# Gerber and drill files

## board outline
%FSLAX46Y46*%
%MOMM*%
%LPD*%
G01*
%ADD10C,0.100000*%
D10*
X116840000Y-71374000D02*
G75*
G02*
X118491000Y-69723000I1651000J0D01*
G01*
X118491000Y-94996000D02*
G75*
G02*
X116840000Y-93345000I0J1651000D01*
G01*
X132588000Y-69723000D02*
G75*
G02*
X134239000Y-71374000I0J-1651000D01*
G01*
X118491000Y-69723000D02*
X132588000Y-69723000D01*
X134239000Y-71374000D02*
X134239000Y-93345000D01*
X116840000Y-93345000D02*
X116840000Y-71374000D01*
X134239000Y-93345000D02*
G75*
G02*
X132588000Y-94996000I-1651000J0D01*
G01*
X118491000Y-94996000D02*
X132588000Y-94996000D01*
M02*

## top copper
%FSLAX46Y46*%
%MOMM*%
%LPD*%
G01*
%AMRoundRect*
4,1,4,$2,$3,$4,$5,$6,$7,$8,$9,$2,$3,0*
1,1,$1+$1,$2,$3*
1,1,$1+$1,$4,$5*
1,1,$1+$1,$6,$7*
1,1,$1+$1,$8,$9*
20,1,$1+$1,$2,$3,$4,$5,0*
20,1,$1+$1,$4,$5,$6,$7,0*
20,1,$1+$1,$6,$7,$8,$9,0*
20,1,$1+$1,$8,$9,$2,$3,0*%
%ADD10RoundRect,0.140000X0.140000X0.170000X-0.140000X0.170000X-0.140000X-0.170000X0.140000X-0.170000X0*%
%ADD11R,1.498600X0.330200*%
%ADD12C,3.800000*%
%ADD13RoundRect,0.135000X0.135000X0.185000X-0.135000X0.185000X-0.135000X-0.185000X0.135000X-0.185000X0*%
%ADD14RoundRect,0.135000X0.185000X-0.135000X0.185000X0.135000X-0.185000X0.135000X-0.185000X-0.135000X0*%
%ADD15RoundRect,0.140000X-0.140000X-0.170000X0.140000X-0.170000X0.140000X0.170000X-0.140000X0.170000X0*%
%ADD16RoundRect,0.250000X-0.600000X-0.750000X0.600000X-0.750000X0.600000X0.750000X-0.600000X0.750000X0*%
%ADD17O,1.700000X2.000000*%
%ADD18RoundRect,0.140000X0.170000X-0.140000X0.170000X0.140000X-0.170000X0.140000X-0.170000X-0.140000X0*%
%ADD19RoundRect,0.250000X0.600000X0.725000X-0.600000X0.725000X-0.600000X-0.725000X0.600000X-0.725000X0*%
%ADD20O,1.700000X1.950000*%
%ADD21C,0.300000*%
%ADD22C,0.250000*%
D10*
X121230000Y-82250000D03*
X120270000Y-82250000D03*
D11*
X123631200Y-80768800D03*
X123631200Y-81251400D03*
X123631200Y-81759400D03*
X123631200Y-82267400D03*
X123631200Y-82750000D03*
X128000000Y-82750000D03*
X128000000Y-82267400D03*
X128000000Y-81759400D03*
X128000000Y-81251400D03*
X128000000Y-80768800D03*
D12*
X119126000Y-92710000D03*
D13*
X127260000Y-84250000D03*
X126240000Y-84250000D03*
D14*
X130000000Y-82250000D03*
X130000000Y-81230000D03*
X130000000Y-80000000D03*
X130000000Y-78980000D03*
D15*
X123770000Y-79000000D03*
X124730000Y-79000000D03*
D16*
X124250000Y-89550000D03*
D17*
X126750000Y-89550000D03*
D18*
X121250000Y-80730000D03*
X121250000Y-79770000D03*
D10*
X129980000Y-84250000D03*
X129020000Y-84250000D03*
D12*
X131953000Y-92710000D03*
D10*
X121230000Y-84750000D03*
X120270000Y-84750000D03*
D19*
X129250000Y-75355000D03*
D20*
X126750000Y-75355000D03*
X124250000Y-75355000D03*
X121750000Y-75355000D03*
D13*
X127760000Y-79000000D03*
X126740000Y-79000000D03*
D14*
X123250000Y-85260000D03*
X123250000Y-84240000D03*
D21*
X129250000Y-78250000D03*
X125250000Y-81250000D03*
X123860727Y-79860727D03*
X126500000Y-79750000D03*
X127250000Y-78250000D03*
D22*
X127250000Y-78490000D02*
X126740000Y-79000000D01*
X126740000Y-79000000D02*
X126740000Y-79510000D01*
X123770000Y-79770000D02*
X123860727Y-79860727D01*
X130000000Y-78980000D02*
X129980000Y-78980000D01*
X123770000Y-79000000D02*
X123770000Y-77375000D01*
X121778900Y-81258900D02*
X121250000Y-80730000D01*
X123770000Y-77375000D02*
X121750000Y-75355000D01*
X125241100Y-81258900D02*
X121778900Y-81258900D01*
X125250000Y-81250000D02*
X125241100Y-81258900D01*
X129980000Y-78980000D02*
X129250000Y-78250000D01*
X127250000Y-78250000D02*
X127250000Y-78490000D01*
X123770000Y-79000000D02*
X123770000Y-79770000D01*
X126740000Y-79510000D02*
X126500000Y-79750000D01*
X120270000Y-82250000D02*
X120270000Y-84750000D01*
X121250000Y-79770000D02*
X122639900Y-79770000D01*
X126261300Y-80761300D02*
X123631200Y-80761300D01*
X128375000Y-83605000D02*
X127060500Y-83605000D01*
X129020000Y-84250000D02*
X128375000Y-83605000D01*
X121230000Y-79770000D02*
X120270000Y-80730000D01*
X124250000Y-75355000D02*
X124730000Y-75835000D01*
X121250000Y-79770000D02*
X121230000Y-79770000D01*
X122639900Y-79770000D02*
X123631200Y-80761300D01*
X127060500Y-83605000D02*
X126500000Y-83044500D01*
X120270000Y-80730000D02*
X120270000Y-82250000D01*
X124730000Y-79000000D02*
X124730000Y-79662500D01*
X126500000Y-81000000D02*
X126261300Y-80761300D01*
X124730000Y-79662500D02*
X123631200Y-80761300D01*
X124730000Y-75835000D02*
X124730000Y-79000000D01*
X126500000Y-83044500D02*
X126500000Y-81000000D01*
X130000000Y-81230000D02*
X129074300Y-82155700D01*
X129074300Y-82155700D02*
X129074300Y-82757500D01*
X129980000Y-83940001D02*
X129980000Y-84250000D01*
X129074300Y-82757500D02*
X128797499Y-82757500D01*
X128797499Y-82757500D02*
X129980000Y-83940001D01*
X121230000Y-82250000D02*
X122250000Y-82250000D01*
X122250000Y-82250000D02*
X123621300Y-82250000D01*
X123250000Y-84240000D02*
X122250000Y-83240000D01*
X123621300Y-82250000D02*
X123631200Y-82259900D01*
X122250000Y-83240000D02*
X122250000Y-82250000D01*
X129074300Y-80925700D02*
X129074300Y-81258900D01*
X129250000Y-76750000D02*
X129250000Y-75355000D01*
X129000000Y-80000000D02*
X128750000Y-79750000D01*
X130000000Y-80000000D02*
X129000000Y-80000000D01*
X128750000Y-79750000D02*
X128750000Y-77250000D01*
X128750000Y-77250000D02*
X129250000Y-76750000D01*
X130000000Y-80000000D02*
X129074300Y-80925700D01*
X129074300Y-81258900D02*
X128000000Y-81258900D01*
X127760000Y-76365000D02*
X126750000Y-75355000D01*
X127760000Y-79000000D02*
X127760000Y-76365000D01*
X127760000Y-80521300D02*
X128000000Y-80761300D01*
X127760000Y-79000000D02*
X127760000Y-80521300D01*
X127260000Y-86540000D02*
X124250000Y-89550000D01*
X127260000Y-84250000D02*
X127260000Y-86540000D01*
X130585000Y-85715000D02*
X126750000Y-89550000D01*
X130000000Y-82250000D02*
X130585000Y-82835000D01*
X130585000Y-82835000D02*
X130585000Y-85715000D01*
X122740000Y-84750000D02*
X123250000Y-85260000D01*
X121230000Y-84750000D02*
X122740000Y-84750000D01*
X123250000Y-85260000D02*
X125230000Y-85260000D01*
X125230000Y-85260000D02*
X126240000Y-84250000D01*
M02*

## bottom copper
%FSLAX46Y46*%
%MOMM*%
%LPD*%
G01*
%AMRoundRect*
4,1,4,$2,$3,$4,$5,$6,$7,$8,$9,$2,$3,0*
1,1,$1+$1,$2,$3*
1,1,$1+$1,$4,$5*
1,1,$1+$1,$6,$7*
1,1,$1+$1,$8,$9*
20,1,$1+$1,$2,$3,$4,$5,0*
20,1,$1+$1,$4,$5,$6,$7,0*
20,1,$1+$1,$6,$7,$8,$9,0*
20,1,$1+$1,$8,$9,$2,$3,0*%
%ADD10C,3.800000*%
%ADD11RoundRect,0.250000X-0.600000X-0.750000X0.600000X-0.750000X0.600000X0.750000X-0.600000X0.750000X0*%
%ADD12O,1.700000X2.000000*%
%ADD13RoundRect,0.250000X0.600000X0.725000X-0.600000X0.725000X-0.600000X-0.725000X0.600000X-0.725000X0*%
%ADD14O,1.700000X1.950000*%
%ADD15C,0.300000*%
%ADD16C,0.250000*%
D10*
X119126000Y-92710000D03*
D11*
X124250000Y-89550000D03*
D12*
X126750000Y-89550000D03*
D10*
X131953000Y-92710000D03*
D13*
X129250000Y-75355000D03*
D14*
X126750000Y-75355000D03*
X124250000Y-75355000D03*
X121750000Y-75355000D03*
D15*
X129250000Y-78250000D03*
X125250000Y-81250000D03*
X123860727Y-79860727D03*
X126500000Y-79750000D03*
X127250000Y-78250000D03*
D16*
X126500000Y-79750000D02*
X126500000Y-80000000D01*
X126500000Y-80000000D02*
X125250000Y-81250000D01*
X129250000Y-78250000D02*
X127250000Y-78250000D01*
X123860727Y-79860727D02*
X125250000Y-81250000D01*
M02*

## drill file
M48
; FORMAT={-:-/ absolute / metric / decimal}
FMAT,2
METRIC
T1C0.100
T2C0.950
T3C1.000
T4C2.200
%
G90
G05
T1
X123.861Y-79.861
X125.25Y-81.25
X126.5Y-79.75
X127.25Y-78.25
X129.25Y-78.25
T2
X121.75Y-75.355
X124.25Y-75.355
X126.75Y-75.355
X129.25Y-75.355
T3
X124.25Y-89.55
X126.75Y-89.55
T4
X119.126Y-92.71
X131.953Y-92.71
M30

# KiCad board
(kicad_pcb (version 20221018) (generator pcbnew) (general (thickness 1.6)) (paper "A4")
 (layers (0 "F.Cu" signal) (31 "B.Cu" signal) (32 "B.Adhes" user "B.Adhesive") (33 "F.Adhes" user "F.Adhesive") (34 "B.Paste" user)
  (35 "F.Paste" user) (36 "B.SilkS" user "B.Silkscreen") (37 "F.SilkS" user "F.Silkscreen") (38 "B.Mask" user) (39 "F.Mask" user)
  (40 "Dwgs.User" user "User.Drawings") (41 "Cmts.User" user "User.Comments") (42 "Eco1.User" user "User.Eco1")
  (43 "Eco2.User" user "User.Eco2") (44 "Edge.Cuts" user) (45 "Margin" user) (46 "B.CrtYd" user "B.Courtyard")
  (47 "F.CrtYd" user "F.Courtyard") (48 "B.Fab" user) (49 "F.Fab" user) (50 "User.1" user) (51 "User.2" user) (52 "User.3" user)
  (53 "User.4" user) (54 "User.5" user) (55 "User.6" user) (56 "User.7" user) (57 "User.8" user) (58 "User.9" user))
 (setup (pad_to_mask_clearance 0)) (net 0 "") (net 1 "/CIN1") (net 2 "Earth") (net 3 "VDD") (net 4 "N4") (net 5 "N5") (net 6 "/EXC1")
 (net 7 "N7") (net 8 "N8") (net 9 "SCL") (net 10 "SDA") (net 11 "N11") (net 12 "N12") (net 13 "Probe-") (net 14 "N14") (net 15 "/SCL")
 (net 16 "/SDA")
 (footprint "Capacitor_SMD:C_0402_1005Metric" (layer "F.Cu") (at 120.75 82.25 180)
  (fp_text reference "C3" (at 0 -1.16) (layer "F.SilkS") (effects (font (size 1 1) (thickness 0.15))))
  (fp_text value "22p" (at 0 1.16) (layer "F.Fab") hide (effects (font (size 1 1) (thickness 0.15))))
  (pad "1" smd roundrect (at -0.48 0 180) (size 0.56 0.62) (layers "F.Cu" "F.Paste" "F.Mask") (roundrect_rratio 0.25) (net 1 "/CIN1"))
  (pad "2" smd roundrect (at 0.48 0 180) (size 0.56 0.62) (layers "F.Cu" "F.Paste" "F.Mask") (roundrect_rratio 0.25) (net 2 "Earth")))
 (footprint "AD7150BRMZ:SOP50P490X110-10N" (layer "F.Cu") (at 125.8156 81.7594)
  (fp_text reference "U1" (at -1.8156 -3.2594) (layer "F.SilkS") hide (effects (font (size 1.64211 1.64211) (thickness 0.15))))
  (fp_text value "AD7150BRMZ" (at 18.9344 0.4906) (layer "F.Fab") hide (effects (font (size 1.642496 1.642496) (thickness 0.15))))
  (pad "1" smd rect (at -2.1844 -0.9906) (size 1.4986 0.3302) (layers "F.Cu" "F.Paste" "F.Mask") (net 2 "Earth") (solder_mask_margin 0.102))
  (pad "2" smd rect (at -2.1844 -0.508) (size 1.4986 0.3302) (layers "F.Cu" "F.Paste" "F.Mask") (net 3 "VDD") (solder_mask_margin 0.102))
  (pad "3" smd rect (at -2.1844 0) (size 1.4986 0.3302) (layers "F.Cu" "F.Paste" "F.Mask") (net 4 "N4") (solder_mask_margin 0.102))
  (pad "4" smd rect (at -2.1844 0.508) (size 1.4986 0.3302) (layers "F.Cu" "F.Paste" "F.Mask") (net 1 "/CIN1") (solder_mask_margin 0.102))
  (pad "5" smd rect (at -2.1844 0.9906) (size 1.4986 0.3302) (layers "F.Cu" "F.Paste" "F.Mask") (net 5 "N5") (solder_mask_margin 0.102))
  (pad "6" smd rect (at 2.1844 0.9906) (size 1.4986 0.3302) (layers "F.Cu" "F.Paste" "F.Mask") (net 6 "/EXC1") (solder_mask_margin 0.102))
  (pad "7" smd rect (at 2.1844 0.508) (size 1.4986 0.3302) (layers "F.Cu" "F.Paste" "F.Mask") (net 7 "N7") (solder_mask_margin 0.102))
  (pad "8" smd rect (at 2.1844 0) (size 1.4986 0.3302) (layers "F.Cu" "F.Paste" "F.Mask") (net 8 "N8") (solder_mask_margin 0.102))
  (pad "9" smd rect (at 2.1844 -0.508) (size 1.4986 0.3302) (layers "F.Cu" "F.Paste" "F.Mask") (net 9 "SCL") (solder_mask_margin 0.102))
  (pad "10" smd rect (at 2.1844 -0.9906) (size 1.4986 0.3302) (layers "F.Cu" "F.Paste" "F.Mask") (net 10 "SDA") (solder_mask_margin 0.102)))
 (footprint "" (layer "F.Cu") (at 119.126 92.71)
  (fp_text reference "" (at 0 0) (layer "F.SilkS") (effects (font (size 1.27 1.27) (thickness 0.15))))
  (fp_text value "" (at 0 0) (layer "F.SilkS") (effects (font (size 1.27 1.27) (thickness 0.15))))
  (pad "1" thru_hole circle (at 0 0 270) (size 3.8 3.8) (drill 2.2) (layers "*.Cu" "*.Mask")))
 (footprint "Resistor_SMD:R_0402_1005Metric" (layer "F.Cu") (at 126.75 84.25 180)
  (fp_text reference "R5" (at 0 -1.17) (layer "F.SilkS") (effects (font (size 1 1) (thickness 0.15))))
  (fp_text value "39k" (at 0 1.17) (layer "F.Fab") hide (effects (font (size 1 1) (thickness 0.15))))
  (pad "1" smd roundrect (at -0.51 0 180) (size 0.54 0.64) (layers "F.Cu" "F.Paste" "F.Mask") (roundrect_rratio 0.25) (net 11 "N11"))
  (pad "2" smd roundrect (at 0.51 0 180) (size 0.54 0.64) (layers "F.Cu" "F.Paste" "F.Mask") (roundrect_rratio 0.25) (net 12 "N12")))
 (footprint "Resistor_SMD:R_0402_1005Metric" (layer "F.Cu") (at 130 81.74 90)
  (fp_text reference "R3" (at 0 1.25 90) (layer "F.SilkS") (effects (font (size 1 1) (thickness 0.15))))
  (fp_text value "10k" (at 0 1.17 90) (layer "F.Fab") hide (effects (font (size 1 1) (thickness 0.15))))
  (pad "1" smd roundrect (at -0.51 0 90) (size 0.54 0.64) (layers "F.Cu" "F.Paste" "F.Mask") (roundrect_rratio 0.25) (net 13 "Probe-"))
  (pad "2" smd roundrect (at 0.51 0 90) (size 0.54 0.64) (layers "F.Cu" "F.Paste" "F.Mask") (roundrect_rratio 0.25) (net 6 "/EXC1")))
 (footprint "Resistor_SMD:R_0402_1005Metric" (layer "F.Cu") (at 130 79.49 90)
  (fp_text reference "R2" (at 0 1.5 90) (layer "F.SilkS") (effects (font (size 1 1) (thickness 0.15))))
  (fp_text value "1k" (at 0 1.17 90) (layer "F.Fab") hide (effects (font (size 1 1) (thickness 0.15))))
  (pad "1" smd roundrect (at -0.51 0 90) (size 0.54 0.64) (layers "F.Cu" "F.Paste" "F.Mask") (roundrect_rratio 0.25) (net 9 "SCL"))
  (pad "2" smd roundrect (at 0.51 0 90) (size 0.54 0.64) (layers "F.Cu" "F.Paste" "F.Mask") (roundrect_rratio 0.25) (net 3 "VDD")))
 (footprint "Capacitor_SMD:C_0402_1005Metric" (layer "F.Cu") (at 124.25 79)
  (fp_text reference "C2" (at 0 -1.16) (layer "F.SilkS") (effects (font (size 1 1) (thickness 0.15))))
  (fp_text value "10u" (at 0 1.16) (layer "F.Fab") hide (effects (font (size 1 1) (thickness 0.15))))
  (pad "1" smd roundrect (at -0.48 0) (size 0.56 0.62) (layers "F.Cu" "F.Paste" "F.Mask") (roundrect_rratio 0.25) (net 3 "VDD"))
  (pad "2" smd roundrect (at 0.48 0) (size 0.56 0.62) (layers "F.Cu" "F.Paste" "F.Mask") (roundrect_rratio 0.25) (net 2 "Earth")))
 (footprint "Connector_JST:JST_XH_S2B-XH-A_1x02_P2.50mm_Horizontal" (layer "F.Cu") (at 124.25 89.55)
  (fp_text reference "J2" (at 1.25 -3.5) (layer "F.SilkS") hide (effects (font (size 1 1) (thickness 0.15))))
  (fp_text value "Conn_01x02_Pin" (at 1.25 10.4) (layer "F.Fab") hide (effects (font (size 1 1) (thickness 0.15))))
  (pad "1" thru_hole roundrect (at 0 0) (size 1.7 2) (drill 1) (layers "*.Cu" "*.Mask") (roundrect_rratio 0.147059) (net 11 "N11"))
  (pad "2" thru_hole oval (at 2.5 0) (size 1.7 2) (drill 1) (layers "*.Cu" "*.Mask") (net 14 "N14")))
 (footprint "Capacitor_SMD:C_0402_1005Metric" (layer "F.Cu") (at 121.25 80.25 90)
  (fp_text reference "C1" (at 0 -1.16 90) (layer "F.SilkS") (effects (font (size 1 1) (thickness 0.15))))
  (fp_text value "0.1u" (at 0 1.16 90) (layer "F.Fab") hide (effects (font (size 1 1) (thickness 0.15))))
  (pad "1" smd roundrect (at -0.48 0 90) (size 0.56 0.62) (layers "F.Cu" "F.Paste" "F.Mask") (roundrect_rratio 0.25) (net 3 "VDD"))
  (pad "2" smd roundrect (at 0.48 0 90) (size 0.56 0.62) (layers "F.Cu" "F.Paste" "F.Mask") (roundrect_rratio 0.25) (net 2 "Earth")))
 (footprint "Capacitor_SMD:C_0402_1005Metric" (layer "F.Cu") (at 129.5 84.25 180)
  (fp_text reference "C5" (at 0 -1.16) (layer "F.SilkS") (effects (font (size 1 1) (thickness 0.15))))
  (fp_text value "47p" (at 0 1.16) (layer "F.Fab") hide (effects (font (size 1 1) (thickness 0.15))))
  (pad "1" smd roundrect (at -0.48 0 180) (size 0.56 0.62) (layers "F.Cu" "F.Paste" "F.Mask") (roundrect_rratio 0.25) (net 6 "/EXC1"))
  (pad "2" smd roundrect (at 0.48 0 180) (size 0.56 0.62) (layers "F.Cu" "F.Paste" "F.Mask") (roundrect_rratio 0.25) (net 2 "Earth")))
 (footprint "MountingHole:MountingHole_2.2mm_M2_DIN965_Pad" (layer "F.Cu") (at 131.953 92.71 -90)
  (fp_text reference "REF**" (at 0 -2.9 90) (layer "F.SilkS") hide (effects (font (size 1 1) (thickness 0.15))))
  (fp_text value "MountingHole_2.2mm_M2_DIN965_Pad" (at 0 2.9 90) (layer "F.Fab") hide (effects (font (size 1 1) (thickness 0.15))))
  (pad "1" thru_hole circle (at 0 0 270) (size 3.8 3.8) (drill 2.2) (layers "*.Cu" "*.Mask")))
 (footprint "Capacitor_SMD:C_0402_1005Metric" (layer "F.Cu") (at 120.75 84.75 180)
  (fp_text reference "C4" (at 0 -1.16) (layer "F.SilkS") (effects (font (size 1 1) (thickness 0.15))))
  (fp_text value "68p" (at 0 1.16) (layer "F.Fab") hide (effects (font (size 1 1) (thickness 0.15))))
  (pad "1" smd roundrect (at -0.48 0 180) (size 0.56 0.62) (layers "F.Cu" "F.Paste" "F.Mask") (roundrect_rratio 0.25) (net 12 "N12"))
  (pad "2" smd roundrect (at 0.48 0 180) (size 0.56 0.62) (layers "F.Cu" "F.Paste" "F.Mask") (roundrect_rratio 0.25) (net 2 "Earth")))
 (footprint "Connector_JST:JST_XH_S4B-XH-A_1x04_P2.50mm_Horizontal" (layer "F.Cu") (at 129.25 75.355 180)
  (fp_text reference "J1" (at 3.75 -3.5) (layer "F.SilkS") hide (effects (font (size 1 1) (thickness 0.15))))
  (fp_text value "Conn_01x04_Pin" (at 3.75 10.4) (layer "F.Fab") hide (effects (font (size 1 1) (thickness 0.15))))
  (pad "1" thru_hole roundrect (at 0 0 180) (size 1.7 1.95) (drill 0.95) (layers "*.Cu" "*.Mask") (roundrect_rratio 0.147059)
   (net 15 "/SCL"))
  (pad "2" thru_hole oval (at 2.5 0 180) (size 1.7 1.95) (drill 0.95) (layers "*.Cu" "*.Mask") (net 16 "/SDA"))
  (pad "3" thru_hole oval (at 5 0 180) (size 1.7 1.95) (drill 0.95) (layers "*.Cu" "*.Mask") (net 2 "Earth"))
  (pad "4" thru_hole oval (at 7.5 0 180) (size 1.7 1.95) (drill 0.95) (layers "*.Cu" "*.Mask") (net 3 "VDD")))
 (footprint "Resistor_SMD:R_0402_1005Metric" (layer "F.Cu") (at 127.25 79 180)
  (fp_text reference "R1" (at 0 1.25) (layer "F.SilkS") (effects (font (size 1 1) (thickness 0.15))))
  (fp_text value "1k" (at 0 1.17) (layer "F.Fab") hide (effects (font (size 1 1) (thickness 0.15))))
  (pad "1" smd roundrect (at -0.51 0 180) (size 0.54 0.64) (layers "F.Cu" "F.Paste" "F.Mask") (roundrect_rratio 0.25) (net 10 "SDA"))
  (pad "2" smd roundrect (at 0.51 0 180) (size 0.54 0.64) (layers "F.Cu" "F.Paste" "F.Mask") (roundrect_rratio 0.25) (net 3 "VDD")))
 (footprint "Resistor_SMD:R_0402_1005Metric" (layer "F.Cu") (at 123.25 84.75 90)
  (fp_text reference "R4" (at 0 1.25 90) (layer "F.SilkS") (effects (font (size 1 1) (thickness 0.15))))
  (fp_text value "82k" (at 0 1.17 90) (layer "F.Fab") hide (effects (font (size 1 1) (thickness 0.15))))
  (pad "1" smd roundrect (at -0.51 0 90) (size 0.54 0.64) (layers "F.Cu" "F.Paste" "F.Mask") (roundrect_rratio 0.25) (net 12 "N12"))
  (pad "2" smd roundrect (at 0.51 0 90) (size 0.54 0.64) (layers "F.Cu" "F.Paste" "F.Mask") (roundrect_rratio 0.25) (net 1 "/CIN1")))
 (gr_arc (start 116.84 71.374) (mid 117.323567 70.206567) (end 118.491 69.723) (stroke (width 0.1) (type default)) (layer "Edge.Cuts"))
 (gr_arc (start 118.491 94.996) (mid 117.323567 94.512433) (end 116.84 93.345) (stroke (width 0.1) (type default)) (layer "Edge.Cuts"))
 (gr_arc (start 132.588 69.723) (mid 133.755433 70.206567) (end 134.239 71.374) (stroke (width 0.1) (type default)) (layer "Edge.Cuts"))
 (gr_line (start 118.491 69.723) (end 132.588 69.723) (stroke (width 0.1) (type default)) (layer "Edge.Cuts"))
 (gr_line (start 134.239 71.374) (end 134.239 93.345) (stroke (width 0.1) (type default)) (layer "Edge.Cuts"))
 (gr_line (start 116.84 93.345) (end 116.84 71.374) (stroke (width 0.1) (type default)) (layer "Edge.Cuts"))
 (gr_arc (start 134.239 93.345) (mid 133.755433 94.512433) (end 132.588 94.996) (stroke (width 0.1) (type default)) (layer "Edge.Cuts"))
 (gr_line (start 118.491 94.996) (end 132.588 94.996) (stroke (width 0.1) (type default)) (layer "Edge.Cuts"))
 (segment (start 127.25 78.49) (end 126.74 79) (width 0.25) (layer "F.Cu") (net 3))
 (segment (start 126.74 79) (end 126.74 79.51) (width 0.25) (layer "F.Cu") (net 3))
 (segment (start 123.77 79.77) (end 123.860727 79.860727) (width 0.25) (layer "F.Cu") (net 3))
 (segment (start 130 78.98) (end 129.98 78.98) (width 0.25) (layer "F.Cu") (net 3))
 (segment (start 123.77 79) (end 123.77 77.375) (width 0.25) (layer "F.Cu") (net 3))
 (segment (start 121.7789 81.2589) (end 121.25 80.73) (width 0.25) (layer "F.Cu") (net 3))
 (segment (start 123.77 77.375) (end 121.75 75.355) (width 0.25) (layer "F.Cu") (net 3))
 (segment (start 125.2411 81.2589) (end 121.7789 81.2589) (width 0.25) (layer "F.Cu") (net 3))
 (segment (start 125.25 81.25) (end 125.2411 81.2589) (width 0.25) (layer "F.Cu") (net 3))
 (segment (start 129.98 78.98) (end 129.25 78.25) (width 0.25) (layer "F.Cu") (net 3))
 (segment (start 127.25 78.25) (end 127.25 78.49) (width 0.25) (layer "F.Cu") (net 3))
 (segment (start 123.77 79) (end 123.77 79.77) (width 0.25) (layer "F.Cu") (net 3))
 (segment (start 126.74 79.51) (end 126.5 79.75) (width 0.25) (layer "F.Cu") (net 3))
 (via micro (at 129.25 78.25) (size 0.3) (drill 0.1) (layers "F.Cu" "B.Cu") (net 3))
 (via micro (at 125.25 81.25) (size 0.3) (drill 0.1) (layers "F.Cu" "B.Cu") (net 3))
 (via micro (at 123.860727 79.860727) (size 0.3) (drill 0.1) (layers "F.Cu" "B.Cu") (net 3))
 (via micro (at 126.5 79.75) (size 0.3) (drill 0.1) (layers "F.Cu" "B.Cu") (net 3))
 (via micro (at 127.25 78.25) (size 0.3) (drill 0.1) (layers "F.Cu" "B.Cu") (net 3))
 (segment (start 126.5 79.75) (end 126.5 80) (width 0.25) (layer "B.Cu") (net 3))
 (segment (start 126.5 80) (end 125.25 81.25) (width 0.25) (layer "B.Cu") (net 3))
 (segment (start 129.25 78.25) (end 127.25 78.25) (width 0.25) (layer "B.Cu") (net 3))
 (segment (start 123.860727 79.860727) (end 125.25 81.25) (width 0.25) (layer "B.Cu") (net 3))
 (segment (start 120.27 82.25) (end 120.27 84.75) (width 0.25) (layer "F.Cu") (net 2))
 (segment (start 121.25 79.77) (end 122.6399 79.77) (width 0.25) (layer "F.Cu") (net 2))
 (segment (start 126.2613 80.7613) (end 123.6312 80.7613) (width 0.25) (layer "F.Cu") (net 2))
 (segment (start 128.375 83.605) (end 127.0605 83.605) (width 0.25) (layer "F.Cu") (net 2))
 (segment (start 129.02 84.25) (end 128.375 83.605) (width 0.25) (layer "F.Cu") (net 2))
 (segment (start 121.23 79.77) (end 120.27 80.73) (width 0.25) (layer "F.Cu") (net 2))
 (segment (start 124.25 75.355) (end 124.73 75.835) (width 0.25) (layer "F.Cu") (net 2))
 (segment (start 121.25 79.77) (end 121.23 79.77) (width 0.25) (layer "F.Cu") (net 2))
 (segment (start 122.6399 79.77) (end 123.6312 80.7613) (width 0.25) (layer "F.Cu") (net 2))
 (segment (start 127.0605 83.605) (end 126.5 83.0445) (width 0.25) (layer "F.Cu") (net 2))
 (segment (start 120.27 80.73) (end 120.27 82.25) (width 0.25) (layer "F.Cu") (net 2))
 (segment (start 124.73 79) (end 124.73 79.6625) (width 0.25) (layer "F.Cu") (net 2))
 (segment (start 126.5 81) (end 126.2613 80.7613) (width 0.25) (layer "F.Cu") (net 2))
 (segment (start 124.73 79.6625) (end 123.6312 80.7613) (width 0.25) (layer "F.Cu") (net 2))
 (segment (start 124.73 75.835) (end 124.73 79) (width 0.25) (layer "F.Cu") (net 2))
 (segment (start 126.5 83.0445) (end 126.5 81) (width 0.25) (layer "F.Cu") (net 2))
 (segment (start 130 81.23) (end 129.0743 82.1557) (width 0.25) (layer "F.Cu") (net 6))
 (segment (start 129.0743 82.1557) (end 129.0743 82.7575) (width 0.25) (layer "F.Cu") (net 6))
 (segment (start 129.98 83.940001) (end 129.98 84.25) (width 0.25) (layer "F.Cu") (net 6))
 (segment (start 129.0743 82.7575) (end 128.797499 82.7575) (width 0.25) (layer "F.Cu") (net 6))
 (segment (start 128.797499 82.7575) (end 129.98 83.940001) (width 0.25) (layer "F.Cu") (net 6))
 (segment (start 121.23 82.25) (end 122.25 82.25) (width 0.25) (layer "F.Cu") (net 1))
 (segment (start 122.25 82.25) (end 123.6213 82.25) (width 0.25) (layer "F.Cu") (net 1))
 (segment (start 123.25 84.24) (end 122.25 83.24) (width 0.25) (layer "F.Cu") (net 1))
 (segment (start 123.6213 82.25) (end 123.6312 82.2599) (width 0.25) (layer "F.Cu") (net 1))
 (segment (start 122.25 83.24) (end 122.25 82.25) (width 0.25) (layer "F.Cu") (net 1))
 (segment (start 129.0743 80.9257) (end 129.0743 81.2589) (width 0.25) (layer "F.Cu") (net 15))
 (segment (start 129.25 76.75) (end 129.25 75.355) (width 0.25) (layer "F.Cu") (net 15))
 (segment (start 129 80) (end 128.75 79.75) (width 0.25) (layer "F.Cu") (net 15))
 (segment (start 130 80) (end 129 80) (width 0.25) (layer "F.Cu") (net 15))
 (segment (start 128.75 79.75) (end 128.75 77.25) (width 0.25) (layer "F.Cu") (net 15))
 (segment (start 128.75 77.25) (end 129.25 76.75) (width 0.25) (layer "F.Cu") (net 15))
 (segment (start 130 80) (end 129.0743 80.9257) (width 0.25) (layer "F.Cu") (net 15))
 (segment (start 129.0743 81.2589) (end 128 81.2589) (width 0.25) (layer "F.Cu") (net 15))
 (segment (start 127.76 76.365) (end 126.75 75.355) (width 0.25) (layer "F.Cu") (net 16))
 (segment (start 127.76 79) (end 127.76 76.365) (width 0.25) (layer "F.Cu") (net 16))
 (segment (start 127.76 80.5213) (end 128 80.7613) (width 0.25) (layer "F.Cu") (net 16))
 (segment (start 127.76 79) (end 127.76 80.5213) (width 0.25) (layer "F.Cu") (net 16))
 (segment (start 127.26 86.54) (end 124.25 89.55) (width 0.25) (layer "F.Cu") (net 11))
 (segment (start 127.26 84.25) (end 127.26 86.54) (width 0.25) (layer "F.Cu") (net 11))
 (segment (start 130.585 85.715) (end 126.75 89.55) (width 0.25) (layer "F.Cu") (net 14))
 (segment (start 130 82.25) (end 130.585 82.835) (width 0.25) (layer "F.Cu") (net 14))
 (segment (start 130.585 82.835) (end 130.585 85.715) (width 0.25) (layer "F.Cu") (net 14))
 (segment (start 122.74 84.75) (end 123.25 85.26) (width 0.25) (layer "F.Cu") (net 12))
 (segment (start 121.23 84.75) (end 122.74 84.75) (width 0.25) (layer "F.Cu") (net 12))
 (segment (start 123.25 85.26) (end 125.23 85.26) (width 0.25) (layer "F.Cu") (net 12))
 (segment (start 125.23 85.26) (end 126.24 84.25) (width 0.25) (layer "F.Cu") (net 12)))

